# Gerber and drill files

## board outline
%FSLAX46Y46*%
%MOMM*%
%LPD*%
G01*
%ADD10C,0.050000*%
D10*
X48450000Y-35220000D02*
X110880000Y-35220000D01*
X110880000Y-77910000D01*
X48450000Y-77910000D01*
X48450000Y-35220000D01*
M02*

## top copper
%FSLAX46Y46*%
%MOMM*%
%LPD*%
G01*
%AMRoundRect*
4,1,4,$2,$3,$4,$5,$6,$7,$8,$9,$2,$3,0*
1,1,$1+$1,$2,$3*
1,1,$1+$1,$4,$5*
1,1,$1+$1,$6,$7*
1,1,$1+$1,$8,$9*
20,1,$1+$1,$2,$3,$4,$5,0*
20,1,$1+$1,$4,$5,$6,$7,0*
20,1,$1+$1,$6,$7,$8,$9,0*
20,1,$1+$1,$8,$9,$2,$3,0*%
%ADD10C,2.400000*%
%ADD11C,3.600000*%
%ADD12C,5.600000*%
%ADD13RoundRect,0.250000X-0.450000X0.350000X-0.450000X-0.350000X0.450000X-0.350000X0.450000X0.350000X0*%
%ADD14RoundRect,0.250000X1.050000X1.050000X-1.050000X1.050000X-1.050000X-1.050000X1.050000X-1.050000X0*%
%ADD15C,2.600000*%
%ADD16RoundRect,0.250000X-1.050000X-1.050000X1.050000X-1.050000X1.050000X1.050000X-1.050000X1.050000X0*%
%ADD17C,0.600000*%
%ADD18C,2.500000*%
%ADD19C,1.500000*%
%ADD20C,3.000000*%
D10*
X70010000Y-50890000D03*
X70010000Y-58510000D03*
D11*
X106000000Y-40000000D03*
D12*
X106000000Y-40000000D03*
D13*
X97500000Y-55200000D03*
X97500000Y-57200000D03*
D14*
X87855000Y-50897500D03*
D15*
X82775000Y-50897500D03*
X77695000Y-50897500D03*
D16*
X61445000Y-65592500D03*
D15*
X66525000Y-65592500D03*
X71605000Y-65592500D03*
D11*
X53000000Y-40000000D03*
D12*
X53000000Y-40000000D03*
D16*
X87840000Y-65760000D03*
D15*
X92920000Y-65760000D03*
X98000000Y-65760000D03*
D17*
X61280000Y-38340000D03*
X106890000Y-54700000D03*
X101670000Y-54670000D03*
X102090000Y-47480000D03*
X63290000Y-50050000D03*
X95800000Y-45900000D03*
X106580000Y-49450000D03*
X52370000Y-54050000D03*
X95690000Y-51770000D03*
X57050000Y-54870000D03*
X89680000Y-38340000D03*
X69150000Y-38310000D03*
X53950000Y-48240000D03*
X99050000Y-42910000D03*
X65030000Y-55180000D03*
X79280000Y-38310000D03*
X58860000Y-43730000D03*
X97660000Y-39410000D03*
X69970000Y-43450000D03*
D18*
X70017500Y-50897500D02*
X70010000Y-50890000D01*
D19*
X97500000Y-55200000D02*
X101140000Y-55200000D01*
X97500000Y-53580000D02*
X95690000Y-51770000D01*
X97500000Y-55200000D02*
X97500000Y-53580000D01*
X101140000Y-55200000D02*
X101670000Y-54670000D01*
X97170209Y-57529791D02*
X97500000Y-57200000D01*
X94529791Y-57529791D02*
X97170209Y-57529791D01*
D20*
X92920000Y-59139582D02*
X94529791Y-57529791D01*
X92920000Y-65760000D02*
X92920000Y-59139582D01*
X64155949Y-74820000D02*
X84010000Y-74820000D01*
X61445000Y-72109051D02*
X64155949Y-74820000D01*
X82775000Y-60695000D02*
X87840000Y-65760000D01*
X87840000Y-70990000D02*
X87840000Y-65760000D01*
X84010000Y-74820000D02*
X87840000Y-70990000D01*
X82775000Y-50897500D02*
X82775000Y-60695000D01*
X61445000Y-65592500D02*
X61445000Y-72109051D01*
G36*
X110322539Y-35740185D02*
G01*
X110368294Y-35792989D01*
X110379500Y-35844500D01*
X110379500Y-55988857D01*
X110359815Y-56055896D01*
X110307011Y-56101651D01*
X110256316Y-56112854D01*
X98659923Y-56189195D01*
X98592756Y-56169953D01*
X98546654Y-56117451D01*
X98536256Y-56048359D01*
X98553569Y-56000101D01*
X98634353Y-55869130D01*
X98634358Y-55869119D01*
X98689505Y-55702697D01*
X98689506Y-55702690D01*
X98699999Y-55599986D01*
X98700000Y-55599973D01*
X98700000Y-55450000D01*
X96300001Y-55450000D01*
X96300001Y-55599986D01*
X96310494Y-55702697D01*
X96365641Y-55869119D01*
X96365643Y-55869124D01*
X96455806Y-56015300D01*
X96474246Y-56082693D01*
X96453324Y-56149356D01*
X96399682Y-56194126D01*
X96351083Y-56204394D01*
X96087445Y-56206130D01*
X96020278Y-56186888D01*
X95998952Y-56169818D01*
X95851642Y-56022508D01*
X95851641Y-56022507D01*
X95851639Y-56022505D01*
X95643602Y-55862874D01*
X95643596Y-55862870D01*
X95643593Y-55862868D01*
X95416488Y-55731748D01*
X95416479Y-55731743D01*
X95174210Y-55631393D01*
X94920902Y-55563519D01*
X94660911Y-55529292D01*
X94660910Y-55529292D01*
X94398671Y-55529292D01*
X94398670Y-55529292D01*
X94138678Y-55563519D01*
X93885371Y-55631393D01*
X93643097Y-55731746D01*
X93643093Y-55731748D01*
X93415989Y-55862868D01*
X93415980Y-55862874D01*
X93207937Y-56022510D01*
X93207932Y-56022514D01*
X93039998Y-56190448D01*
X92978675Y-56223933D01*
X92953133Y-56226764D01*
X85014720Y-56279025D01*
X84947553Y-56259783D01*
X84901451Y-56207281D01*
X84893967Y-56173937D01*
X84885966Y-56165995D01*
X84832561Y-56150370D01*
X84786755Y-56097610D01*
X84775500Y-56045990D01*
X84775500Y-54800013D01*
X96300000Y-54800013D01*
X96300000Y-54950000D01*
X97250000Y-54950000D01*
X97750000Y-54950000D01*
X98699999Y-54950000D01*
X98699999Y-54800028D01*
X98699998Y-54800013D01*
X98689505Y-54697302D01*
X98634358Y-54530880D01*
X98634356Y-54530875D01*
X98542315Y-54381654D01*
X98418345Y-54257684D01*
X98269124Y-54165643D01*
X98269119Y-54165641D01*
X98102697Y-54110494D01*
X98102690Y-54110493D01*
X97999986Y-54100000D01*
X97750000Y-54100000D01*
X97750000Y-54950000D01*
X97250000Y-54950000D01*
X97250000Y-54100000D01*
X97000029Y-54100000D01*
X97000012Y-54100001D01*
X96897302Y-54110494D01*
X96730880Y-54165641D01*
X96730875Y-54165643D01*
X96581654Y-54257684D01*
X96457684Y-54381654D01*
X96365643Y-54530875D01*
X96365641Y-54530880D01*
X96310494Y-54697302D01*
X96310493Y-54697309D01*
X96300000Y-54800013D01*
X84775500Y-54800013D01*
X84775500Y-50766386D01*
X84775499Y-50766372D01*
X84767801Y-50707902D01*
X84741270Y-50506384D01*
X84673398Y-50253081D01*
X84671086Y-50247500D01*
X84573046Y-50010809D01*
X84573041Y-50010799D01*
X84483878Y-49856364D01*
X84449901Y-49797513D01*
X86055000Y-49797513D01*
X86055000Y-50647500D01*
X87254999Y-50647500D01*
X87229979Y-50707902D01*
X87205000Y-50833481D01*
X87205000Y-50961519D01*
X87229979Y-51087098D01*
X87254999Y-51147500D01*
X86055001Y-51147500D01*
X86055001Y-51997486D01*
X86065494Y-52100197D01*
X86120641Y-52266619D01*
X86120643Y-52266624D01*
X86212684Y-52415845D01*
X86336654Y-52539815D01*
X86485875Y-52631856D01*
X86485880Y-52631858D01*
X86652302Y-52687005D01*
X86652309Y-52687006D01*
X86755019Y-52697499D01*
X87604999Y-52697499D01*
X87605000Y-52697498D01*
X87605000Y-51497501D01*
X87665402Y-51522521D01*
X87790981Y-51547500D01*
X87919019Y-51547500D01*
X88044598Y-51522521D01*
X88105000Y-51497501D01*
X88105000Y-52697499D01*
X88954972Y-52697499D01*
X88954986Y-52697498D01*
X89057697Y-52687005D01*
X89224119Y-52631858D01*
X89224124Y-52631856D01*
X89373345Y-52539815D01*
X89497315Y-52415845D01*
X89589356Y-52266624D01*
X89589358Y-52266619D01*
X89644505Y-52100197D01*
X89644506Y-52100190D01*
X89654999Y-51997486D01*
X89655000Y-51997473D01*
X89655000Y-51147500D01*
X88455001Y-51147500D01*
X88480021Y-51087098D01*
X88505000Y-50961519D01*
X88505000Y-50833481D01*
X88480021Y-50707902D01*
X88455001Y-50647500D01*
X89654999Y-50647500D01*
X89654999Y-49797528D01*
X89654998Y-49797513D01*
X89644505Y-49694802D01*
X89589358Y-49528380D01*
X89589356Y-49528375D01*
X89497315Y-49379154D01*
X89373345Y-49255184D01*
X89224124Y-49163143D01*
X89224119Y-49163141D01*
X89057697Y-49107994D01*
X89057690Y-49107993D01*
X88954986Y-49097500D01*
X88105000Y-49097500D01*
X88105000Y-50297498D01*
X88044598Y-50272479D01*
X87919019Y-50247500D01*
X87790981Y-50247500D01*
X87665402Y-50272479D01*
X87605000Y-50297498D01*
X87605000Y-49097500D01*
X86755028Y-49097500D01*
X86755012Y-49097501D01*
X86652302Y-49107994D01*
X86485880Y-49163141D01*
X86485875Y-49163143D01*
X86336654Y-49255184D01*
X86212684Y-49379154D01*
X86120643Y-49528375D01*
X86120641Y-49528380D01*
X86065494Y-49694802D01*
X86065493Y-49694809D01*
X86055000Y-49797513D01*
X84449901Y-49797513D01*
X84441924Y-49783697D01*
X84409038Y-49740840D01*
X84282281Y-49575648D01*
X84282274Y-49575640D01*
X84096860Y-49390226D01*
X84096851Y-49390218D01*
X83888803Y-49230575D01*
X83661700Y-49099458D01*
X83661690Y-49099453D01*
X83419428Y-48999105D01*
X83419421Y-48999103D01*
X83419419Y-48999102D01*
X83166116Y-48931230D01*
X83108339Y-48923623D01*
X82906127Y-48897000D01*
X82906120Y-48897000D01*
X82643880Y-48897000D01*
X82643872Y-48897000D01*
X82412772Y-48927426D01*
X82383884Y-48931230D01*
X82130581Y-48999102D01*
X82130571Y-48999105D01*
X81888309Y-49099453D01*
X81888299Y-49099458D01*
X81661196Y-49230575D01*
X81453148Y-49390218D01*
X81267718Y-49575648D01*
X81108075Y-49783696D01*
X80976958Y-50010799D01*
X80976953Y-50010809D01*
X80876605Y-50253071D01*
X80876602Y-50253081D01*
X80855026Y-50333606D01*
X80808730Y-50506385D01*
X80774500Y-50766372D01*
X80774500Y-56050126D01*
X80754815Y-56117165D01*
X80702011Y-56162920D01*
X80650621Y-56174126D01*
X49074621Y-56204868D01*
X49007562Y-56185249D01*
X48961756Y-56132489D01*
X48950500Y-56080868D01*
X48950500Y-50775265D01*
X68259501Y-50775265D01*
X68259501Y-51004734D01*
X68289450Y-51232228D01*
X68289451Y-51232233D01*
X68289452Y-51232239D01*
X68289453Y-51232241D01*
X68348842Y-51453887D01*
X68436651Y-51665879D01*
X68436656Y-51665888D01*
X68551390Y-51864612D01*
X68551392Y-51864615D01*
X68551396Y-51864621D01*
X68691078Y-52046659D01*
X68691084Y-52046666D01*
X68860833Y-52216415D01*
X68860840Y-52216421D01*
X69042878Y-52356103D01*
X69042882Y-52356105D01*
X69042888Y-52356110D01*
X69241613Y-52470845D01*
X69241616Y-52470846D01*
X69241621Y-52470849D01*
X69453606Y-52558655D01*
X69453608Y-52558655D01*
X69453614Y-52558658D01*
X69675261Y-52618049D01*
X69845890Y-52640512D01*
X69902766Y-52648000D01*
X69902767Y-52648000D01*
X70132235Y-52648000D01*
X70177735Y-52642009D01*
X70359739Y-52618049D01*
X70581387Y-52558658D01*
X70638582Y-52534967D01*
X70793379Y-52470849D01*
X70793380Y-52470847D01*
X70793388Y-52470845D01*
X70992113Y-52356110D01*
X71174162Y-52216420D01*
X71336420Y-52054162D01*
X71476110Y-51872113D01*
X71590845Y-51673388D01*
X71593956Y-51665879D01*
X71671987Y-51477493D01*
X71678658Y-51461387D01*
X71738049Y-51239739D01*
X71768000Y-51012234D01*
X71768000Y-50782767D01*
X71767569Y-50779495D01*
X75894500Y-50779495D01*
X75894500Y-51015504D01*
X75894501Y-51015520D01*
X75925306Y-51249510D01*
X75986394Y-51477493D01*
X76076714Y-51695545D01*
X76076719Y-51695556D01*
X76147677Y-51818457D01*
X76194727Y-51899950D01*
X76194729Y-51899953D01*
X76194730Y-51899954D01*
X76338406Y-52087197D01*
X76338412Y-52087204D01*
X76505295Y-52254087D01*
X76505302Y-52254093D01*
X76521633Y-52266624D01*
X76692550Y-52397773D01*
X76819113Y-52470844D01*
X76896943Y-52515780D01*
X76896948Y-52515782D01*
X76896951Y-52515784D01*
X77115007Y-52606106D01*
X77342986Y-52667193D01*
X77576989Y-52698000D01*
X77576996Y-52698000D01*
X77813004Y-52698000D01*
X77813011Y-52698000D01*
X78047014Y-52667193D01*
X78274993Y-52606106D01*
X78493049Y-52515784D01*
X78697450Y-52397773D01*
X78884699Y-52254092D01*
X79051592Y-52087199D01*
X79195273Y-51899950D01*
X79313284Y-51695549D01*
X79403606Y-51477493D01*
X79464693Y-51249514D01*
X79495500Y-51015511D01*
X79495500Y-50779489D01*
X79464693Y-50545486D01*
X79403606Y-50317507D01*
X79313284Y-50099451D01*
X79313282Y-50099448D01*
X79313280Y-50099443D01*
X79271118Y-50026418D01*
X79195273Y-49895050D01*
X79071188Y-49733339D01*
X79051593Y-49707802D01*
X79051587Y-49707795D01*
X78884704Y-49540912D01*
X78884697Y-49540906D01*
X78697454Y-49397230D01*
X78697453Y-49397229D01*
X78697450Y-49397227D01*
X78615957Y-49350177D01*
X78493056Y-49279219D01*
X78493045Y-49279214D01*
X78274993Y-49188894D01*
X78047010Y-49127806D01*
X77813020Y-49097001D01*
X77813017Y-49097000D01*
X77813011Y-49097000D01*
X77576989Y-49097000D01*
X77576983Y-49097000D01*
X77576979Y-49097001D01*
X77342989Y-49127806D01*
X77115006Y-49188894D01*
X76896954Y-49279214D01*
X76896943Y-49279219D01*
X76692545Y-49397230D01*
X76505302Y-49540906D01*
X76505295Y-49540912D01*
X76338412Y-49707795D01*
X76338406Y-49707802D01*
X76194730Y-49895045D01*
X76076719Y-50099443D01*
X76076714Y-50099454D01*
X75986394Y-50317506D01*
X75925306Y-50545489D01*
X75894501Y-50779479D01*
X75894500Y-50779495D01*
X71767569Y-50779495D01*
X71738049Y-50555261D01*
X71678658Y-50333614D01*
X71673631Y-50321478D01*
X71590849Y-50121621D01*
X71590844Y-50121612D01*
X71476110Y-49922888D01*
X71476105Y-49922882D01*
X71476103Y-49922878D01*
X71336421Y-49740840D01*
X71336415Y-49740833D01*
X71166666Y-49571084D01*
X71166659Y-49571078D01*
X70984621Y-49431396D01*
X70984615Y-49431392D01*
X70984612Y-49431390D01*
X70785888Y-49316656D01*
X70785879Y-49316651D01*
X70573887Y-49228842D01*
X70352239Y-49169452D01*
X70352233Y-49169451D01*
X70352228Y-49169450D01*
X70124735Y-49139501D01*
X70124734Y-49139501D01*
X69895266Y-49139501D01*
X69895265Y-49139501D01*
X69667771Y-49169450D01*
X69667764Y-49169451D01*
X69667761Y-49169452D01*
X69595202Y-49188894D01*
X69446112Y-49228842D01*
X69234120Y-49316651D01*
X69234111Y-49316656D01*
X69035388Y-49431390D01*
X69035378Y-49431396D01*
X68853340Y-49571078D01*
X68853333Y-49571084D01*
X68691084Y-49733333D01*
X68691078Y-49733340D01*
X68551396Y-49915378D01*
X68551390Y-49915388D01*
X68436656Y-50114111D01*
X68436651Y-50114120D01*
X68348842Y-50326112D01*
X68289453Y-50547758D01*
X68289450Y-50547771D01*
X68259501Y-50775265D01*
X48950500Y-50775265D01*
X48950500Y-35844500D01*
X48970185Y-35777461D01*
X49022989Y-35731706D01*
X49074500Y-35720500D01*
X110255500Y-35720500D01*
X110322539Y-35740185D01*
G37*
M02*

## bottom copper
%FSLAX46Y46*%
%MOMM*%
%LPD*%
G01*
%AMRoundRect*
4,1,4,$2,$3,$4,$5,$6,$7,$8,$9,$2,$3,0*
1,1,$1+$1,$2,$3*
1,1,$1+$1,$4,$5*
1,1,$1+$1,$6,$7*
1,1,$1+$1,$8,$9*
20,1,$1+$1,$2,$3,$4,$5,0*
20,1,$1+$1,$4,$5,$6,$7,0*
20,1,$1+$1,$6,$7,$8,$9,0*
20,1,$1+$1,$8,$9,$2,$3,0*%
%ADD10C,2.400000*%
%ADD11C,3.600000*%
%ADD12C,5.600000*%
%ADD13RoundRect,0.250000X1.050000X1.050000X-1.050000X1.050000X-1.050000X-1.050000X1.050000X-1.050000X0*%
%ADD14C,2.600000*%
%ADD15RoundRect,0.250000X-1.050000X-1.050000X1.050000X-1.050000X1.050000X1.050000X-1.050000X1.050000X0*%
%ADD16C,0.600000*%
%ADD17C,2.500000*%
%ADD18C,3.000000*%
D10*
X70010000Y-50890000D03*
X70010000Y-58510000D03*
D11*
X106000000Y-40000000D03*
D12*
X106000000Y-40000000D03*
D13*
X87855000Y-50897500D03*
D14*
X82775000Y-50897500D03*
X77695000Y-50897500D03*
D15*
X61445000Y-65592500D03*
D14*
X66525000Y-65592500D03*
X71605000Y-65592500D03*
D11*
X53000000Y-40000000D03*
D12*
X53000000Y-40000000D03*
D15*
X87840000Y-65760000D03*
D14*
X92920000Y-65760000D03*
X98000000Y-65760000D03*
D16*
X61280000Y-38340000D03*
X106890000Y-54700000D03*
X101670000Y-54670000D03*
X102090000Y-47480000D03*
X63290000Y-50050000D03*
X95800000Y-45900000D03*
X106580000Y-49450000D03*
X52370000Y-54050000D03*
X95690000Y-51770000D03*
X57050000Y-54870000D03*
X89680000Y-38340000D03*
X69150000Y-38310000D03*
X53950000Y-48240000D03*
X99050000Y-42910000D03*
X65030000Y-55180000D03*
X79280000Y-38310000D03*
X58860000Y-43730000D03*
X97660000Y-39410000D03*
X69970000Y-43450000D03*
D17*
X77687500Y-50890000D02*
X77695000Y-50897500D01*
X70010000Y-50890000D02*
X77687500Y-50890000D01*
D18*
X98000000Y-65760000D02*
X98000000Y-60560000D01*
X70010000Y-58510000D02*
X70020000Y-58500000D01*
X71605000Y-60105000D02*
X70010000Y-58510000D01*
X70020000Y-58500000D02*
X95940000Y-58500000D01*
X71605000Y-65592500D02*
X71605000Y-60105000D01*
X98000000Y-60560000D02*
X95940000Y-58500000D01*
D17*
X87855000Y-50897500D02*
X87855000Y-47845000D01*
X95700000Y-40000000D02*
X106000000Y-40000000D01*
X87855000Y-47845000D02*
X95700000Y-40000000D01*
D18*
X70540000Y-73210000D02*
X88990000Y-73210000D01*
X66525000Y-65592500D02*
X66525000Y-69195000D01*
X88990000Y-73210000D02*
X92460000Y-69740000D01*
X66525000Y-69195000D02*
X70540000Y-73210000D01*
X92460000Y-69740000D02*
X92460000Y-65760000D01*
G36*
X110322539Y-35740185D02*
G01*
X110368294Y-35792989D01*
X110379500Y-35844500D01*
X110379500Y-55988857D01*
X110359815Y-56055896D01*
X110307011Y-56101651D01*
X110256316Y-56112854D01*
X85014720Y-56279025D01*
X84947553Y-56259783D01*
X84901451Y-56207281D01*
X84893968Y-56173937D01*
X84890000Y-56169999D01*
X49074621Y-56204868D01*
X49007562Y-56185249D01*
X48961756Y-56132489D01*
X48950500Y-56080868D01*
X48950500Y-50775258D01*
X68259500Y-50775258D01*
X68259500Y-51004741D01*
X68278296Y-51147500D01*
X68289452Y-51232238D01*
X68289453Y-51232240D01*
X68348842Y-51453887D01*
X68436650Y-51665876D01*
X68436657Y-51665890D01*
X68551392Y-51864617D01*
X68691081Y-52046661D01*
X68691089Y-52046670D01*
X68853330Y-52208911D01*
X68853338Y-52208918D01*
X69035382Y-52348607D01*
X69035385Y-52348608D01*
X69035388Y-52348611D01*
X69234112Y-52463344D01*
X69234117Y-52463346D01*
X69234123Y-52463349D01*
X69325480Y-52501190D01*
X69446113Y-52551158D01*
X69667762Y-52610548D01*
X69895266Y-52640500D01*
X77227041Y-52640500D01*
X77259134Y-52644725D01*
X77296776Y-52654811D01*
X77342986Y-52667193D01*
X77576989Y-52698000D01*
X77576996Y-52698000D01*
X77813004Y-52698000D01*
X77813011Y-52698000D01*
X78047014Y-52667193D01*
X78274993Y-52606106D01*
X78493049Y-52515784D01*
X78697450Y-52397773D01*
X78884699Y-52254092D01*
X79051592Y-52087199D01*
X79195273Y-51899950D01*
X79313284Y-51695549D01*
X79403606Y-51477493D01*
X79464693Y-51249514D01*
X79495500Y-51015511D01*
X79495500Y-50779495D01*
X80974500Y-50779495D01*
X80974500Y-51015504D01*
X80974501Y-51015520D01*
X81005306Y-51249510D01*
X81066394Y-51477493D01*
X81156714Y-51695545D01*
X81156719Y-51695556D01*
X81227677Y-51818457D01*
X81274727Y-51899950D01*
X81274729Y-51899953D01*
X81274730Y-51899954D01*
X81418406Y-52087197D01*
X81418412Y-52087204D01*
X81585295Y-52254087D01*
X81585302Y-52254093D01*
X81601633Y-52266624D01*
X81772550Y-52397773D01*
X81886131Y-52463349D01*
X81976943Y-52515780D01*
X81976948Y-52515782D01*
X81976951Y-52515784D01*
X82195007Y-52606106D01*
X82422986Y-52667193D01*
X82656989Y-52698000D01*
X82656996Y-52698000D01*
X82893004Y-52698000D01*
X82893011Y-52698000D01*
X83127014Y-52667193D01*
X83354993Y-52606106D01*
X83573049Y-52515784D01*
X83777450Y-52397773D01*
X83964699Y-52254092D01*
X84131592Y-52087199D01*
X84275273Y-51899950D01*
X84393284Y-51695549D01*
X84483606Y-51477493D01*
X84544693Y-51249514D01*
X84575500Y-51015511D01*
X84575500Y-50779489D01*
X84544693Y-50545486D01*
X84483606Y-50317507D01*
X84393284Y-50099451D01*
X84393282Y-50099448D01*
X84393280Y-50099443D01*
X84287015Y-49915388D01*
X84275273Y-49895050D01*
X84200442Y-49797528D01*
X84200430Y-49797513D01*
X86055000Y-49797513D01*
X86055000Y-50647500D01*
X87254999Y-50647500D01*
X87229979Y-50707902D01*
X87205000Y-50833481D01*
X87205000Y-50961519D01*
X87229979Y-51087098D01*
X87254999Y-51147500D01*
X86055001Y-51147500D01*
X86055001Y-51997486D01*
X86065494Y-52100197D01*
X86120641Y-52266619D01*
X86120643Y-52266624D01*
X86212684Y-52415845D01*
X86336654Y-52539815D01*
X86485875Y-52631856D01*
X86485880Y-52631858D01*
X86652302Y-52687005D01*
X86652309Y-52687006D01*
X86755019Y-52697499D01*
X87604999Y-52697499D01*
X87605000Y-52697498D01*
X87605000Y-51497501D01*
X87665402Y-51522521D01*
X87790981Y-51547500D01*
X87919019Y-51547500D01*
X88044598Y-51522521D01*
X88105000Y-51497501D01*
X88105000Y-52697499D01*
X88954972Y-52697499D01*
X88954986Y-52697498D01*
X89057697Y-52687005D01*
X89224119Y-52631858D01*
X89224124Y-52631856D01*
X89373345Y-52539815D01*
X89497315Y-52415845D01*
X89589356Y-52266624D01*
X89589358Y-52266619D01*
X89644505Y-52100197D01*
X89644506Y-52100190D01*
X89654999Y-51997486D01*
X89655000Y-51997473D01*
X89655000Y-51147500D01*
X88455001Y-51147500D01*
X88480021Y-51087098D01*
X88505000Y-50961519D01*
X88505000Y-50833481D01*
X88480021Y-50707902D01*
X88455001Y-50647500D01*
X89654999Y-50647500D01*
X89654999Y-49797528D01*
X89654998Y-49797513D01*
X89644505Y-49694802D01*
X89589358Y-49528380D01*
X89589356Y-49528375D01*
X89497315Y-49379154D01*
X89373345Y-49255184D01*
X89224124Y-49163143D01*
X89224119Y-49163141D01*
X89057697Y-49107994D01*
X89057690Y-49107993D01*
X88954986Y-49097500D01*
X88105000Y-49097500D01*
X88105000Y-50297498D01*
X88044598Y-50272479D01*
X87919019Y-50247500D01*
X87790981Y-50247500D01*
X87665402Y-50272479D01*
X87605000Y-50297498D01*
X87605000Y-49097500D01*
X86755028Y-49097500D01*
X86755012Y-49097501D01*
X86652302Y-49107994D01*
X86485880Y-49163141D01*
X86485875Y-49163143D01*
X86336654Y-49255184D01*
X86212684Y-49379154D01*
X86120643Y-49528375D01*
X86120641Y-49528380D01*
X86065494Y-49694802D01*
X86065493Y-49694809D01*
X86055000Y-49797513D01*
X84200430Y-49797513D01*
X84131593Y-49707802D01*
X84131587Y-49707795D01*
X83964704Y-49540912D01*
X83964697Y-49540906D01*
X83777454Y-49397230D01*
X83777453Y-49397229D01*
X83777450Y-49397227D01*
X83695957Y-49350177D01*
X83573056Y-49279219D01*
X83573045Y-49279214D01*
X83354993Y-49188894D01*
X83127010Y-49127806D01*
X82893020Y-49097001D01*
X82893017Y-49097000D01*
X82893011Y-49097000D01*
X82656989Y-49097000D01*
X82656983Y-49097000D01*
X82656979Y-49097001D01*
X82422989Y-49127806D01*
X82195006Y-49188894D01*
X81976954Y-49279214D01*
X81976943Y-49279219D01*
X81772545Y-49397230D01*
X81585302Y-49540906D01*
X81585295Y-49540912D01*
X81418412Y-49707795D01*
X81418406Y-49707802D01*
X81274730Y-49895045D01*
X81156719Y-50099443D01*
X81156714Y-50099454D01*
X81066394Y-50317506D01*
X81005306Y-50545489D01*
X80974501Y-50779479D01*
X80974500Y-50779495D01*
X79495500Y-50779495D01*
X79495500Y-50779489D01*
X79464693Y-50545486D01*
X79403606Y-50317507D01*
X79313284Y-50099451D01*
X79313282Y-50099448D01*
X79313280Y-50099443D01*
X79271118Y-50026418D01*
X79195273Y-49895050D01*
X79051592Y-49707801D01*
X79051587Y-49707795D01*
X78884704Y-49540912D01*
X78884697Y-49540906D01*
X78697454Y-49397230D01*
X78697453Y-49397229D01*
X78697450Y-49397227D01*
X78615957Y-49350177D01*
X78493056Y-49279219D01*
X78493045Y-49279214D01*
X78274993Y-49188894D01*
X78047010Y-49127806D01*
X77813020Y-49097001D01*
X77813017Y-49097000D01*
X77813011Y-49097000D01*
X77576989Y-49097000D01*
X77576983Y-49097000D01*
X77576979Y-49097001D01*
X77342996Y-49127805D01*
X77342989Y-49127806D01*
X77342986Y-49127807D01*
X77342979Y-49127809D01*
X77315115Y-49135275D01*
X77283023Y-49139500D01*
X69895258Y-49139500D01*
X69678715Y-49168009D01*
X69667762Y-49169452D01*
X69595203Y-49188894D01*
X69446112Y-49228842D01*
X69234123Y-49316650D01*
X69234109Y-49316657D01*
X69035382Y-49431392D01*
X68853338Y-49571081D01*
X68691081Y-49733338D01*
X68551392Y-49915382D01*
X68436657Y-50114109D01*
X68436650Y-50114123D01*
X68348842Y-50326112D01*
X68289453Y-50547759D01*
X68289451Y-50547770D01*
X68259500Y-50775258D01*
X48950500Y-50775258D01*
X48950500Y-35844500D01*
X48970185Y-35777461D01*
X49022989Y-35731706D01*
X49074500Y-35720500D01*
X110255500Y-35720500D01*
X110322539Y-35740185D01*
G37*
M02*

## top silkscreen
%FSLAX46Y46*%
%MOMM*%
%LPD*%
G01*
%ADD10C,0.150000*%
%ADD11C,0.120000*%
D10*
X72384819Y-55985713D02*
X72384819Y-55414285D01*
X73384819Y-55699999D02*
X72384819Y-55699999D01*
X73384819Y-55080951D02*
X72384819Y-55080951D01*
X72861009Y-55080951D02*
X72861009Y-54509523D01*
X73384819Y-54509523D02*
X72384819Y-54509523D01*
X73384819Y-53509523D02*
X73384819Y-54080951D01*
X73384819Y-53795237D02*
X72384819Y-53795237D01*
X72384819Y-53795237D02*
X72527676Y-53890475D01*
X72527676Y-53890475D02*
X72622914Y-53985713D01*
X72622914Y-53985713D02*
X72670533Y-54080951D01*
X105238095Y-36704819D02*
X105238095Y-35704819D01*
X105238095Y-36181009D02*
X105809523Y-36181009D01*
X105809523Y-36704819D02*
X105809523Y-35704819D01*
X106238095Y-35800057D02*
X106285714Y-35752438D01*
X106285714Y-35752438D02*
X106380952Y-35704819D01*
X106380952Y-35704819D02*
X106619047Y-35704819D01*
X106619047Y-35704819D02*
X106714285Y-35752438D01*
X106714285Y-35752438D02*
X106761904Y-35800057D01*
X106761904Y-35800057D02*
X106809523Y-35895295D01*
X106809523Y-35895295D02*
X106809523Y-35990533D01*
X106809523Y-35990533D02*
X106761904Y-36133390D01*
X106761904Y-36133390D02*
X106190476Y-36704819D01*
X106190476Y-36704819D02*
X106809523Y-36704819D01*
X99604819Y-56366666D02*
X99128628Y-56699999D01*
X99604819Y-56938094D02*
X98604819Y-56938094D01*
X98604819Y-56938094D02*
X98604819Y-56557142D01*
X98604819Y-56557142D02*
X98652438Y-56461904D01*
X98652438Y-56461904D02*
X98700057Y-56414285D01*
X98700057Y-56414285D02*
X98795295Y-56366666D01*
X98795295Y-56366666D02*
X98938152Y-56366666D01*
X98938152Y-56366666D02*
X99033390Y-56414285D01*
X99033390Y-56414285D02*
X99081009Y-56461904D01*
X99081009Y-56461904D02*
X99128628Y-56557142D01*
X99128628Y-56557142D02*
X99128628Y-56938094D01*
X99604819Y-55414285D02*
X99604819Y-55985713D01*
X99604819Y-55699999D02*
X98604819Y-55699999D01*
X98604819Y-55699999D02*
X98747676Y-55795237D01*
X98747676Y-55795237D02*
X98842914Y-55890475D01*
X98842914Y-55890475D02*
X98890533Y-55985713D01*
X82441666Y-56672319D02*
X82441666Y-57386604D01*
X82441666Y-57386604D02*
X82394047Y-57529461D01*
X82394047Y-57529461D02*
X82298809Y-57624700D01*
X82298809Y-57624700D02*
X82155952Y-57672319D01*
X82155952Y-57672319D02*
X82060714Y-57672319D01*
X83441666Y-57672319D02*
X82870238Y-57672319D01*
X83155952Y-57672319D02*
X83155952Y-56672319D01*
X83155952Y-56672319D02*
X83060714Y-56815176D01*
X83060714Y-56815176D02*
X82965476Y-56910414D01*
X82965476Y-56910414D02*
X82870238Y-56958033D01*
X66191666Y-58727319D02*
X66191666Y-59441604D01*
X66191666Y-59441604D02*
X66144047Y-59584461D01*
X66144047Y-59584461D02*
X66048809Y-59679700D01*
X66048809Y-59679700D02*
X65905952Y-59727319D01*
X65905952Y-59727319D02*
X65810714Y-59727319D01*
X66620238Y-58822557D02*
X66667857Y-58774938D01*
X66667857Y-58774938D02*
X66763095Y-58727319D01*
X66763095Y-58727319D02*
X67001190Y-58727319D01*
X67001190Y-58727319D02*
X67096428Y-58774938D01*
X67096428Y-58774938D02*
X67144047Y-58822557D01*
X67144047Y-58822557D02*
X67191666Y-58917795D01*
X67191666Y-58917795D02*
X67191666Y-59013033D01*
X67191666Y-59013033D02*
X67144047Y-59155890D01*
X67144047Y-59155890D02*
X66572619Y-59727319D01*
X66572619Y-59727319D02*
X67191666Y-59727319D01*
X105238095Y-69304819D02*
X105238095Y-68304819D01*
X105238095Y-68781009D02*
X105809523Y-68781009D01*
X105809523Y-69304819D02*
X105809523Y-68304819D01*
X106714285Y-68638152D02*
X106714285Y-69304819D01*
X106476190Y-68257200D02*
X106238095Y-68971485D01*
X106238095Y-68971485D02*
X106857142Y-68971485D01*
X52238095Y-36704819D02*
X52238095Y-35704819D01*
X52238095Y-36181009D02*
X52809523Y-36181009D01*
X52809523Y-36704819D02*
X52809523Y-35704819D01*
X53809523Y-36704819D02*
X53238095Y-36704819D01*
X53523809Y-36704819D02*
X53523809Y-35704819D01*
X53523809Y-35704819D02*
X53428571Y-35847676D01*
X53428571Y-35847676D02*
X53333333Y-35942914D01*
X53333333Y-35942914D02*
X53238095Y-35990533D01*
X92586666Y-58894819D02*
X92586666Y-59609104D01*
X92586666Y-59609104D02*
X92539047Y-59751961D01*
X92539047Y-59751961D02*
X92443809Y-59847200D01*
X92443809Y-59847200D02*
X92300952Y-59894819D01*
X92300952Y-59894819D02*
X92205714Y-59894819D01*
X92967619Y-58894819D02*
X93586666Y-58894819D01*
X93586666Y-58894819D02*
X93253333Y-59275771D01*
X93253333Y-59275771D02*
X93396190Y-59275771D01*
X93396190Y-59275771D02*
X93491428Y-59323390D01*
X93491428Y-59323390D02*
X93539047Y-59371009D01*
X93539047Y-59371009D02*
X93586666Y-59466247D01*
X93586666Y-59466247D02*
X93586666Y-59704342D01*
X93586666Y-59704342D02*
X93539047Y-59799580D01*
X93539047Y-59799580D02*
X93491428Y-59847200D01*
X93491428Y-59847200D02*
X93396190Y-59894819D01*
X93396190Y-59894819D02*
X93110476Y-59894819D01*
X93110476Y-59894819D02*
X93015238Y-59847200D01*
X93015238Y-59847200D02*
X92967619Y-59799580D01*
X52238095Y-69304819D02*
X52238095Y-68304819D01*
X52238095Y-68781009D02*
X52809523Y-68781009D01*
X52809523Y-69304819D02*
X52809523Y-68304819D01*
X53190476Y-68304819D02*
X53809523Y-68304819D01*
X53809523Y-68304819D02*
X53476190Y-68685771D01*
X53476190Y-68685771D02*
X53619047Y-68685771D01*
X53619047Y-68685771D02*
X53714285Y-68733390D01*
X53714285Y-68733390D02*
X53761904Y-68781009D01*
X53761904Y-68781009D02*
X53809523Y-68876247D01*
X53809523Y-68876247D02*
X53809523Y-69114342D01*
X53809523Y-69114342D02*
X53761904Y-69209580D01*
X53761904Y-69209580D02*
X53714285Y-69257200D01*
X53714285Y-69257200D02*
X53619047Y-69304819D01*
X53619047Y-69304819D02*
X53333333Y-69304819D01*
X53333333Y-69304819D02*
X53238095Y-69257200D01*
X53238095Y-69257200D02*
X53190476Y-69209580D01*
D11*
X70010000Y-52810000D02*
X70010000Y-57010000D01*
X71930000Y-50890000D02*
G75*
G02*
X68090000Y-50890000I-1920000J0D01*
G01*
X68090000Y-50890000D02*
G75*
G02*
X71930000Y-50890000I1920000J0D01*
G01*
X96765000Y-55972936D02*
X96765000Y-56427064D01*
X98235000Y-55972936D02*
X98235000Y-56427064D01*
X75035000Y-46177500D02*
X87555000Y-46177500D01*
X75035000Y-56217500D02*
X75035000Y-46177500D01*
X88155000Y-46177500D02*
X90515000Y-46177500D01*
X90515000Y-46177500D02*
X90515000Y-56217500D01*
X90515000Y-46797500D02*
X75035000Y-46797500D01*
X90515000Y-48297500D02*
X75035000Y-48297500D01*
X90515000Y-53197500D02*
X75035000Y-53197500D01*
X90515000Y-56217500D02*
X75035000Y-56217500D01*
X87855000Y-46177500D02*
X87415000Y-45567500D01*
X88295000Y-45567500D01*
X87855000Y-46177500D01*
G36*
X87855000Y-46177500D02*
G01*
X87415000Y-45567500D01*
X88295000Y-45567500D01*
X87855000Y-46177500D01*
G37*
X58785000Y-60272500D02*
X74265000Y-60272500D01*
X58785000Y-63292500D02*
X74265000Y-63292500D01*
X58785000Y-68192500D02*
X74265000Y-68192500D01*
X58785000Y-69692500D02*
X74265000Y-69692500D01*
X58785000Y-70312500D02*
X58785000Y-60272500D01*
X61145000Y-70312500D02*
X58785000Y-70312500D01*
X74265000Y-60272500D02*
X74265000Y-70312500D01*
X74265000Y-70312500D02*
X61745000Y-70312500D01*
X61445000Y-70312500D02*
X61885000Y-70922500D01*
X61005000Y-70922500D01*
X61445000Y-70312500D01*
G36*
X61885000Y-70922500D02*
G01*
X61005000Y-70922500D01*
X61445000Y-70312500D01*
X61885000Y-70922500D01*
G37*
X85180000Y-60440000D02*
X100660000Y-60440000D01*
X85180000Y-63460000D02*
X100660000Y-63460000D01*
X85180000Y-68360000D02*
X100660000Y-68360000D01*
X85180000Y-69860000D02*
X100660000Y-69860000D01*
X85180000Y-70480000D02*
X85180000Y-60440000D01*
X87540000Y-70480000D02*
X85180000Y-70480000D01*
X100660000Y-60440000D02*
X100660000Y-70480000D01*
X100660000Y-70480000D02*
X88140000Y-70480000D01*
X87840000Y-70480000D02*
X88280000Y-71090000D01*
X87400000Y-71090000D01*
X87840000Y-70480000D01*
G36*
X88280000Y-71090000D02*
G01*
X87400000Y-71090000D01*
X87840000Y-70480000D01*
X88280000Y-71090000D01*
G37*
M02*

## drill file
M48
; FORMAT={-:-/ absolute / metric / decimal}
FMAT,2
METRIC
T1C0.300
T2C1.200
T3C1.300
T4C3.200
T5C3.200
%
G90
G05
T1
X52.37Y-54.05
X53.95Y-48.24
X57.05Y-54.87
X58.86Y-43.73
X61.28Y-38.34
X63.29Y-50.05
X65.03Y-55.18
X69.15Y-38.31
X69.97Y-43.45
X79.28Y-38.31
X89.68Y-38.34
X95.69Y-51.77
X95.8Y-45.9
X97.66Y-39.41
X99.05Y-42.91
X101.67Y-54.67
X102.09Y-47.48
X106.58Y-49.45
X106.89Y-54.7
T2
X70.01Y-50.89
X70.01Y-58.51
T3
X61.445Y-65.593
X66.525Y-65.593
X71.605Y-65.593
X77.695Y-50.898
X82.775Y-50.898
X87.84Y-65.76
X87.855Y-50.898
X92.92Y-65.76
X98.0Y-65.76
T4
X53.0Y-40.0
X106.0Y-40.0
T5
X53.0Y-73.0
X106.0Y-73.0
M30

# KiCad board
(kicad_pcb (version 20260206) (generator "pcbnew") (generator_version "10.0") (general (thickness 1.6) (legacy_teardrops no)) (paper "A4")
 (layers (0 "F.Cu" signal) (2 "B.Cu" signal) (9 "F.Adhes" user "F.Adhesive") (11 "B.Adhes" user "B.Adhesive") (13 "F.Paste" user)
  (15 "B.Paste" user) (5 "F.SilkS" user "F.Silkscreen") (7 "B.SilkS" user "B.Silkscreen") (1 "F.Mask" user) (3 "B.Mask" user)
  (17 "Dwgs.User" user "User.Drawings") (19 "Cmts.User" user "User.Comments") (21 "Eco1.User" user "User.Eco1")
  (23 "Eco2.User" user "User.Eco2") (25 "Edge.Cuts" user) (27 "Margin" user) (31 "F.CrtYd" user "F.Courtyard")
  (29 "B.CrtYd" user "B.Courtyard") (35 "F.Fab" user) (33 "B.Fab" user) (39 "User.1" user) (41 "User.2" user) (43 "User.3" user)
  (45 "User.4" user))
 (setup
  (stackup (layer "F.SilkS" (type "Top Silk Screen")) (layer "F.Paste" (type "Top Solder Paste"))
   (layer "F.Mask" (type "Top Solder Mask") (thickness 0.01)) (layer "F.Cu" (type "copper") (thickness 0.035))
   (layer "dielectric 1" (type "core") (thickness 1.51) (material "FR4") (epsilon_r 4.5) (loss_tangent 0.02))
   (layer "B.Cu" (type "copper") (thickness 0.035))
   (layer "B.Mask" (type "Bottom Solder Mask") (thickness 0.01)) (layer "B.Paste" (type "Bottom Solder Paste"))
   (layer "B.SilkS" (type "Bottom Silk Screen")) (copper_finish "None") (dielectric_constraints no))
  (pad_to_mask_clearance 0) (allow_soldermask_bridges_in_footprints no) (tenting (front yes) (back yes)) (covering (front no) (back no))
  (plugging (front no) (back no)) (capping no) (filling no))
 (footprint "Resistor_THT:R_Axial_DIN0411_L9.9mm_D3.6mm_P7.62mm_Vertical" (layer "F.Cu") (at 70.01 50.89 -90)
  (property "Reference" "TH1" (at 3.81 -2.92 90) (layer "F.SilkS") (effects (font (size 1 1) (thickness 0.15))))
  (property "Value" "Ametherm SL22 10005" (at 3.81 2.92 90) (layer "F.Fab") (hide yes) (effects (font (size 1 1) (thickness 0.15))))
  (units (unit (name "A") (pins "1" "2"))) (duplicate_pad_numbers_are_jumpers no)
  (fp_line (start 1.92 0) (end 6.12 0) (stroke (width 0.12) (type solid)) (layer "F.SilkS"))
  (fp_circle (center 0 0) (end 1.92 0) (stroke (width 0.12) (type solid)) (fill no) (layer "F.SilkS"))
  (pad "1" thru_hole circle (at 0 0 270) (size 2.4 2.4) (drill 1.2) (layers "*.Cu" "*.Mask") (remove_unused_layers no) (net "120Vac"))
  (pad "2" thru_hole circle (at 7.62 0 270) (size 2.4 2.4) (drill 1.2) (layers "*.Cu" "*.Mask") (remove_unused_layers no) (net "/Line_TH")))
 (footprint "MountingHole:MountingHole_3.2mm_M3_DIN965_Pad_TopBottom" (layer "F.Cu") (at 106 40)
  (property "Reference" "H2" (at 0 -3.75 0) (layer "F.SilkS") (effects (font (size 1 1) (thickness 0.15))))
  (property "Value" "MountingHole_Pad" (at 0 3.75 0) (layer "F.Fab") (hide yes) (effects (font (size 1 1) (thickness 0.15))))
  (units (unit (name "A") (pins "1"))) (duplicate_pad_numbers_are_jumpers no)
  (pad "1" thru_hole circle (at 0 0) (size 3.6 3.6) (drill 3.2) (layers "*.Cu" "*.Mask") (remove_unused_layers no) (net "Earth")
   (zone_connect 2))
  (pad "1" connect circle (at 0 0) (size 5.6 5.6) (layers "F.Cu" "F.Mask") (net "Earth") (zone_connect 2))
  (pad "1" connect circle (at 0 0) (size 5.6 5.6) (layers "B.Cu" "B.Mask") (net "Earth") (zone_connect 2)))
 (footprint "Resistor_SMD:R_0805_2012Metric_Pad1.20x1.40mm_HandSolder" (layer "F.Cu") (at 97.5 56.2 -90)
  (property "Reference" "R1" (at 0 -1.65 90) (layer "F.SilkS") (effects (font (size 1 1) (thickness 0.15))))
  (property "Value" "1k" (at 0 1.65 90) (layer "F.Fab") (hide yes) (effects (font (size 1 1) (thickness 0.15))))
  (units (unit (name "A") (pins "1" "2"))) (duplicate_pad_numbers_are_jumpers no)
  (fp_line (start -0.227064 0.735) (end 0.227064 0.735) (stroke (width 0.12) (type solid)) (layer "F.SilkS"))
  (fp_line (start -0.227064 -0.735) (end 0.227064 -0.735) (stroke (width 0.12) (type solid)) (layer "F.SilkS"))
  (pad "1" smd roundrect (at -1 0 270) (size 1.2 1.4) (layers "F.Cu" "F.Mask" "F.Paste") (roundrect_rratio 0.208333) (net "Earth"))
  (pad "2" smd roundrect (at 1 0 270) (size 1.2 1.4) (layers "F.Cu" "F.Mask" "F.Paste") (roundrect_rratio 0.208333) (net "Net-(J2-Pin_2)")))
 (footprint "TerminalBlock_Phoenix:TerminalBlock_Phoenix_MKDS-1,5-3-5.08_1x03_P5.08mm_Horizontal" (layer "F.Cu") (at 87.855 50.8975 180)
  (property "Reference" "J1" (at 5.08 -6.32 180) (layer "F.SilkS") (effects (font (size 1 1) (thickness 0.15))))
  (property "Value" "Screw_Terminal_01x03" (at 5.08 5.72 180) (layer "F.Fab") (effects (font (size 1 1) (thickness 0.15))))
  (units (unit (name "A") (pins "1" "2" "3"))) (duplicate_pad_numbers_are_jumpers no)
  (fp_line (start 12.82 4.72) (end 0.3 4.72) (stroke (width 0.12) (type solid)) (layer "F.SilkS"))
  (fp_line (start 12.82 -5.32) (end 12.82 4.72) (stroke (width 0.12) (type solid)) (layer "F.SilkS"))
  (fp_line (start -0.3 4.72) (end -2.66 4.72) (stroke (width 0.12) (type solid)) (layer "F.SilkS"))
  (fp_line (start -2.66 4.72) (end -2.66 -5.32) (stroke (width 0.12) (type solid)) (layer "F.SilkS"))
  (fp_line (start -2.66 4.1) (end 12.82 4.1) (stroke (width 0.12) (type solid)) (layer "F.SilkS"))
  (fp_line (start -2.66 2.6) (end 12.82 2.6) (stroke (width 0.12) (type solid)) (layer "F.SilkS"))
  (fp_line (start -2.66 -2.3) (end 12.82 -2.3) (stroke (width 0.12) (type solid)) (layer "F.SilkS"))
  (fp_line (start -2.66 -5.32) (end 12.82 -5.32) (stroke (width 0.12) (type solid)) (layer "F.SilkS"))
  (fp_poly (pts (xy 0 4.72) (xy 0.44 5.33) (xy -0.44 5.33)) (stroke (width 0.12) (type solid)) (fill yes) (layer "F.SilkS"))
  (pad "1" thru_hole roundrect (at 0 0 180) (size 2.6 2.6) (drill 1.3) (layers "*.Cu" "*.Mask") (remove_unused_layers no)
   (roundrect_rratio 0.096154) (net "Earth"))
  (pad "2" thru_hole circle (at 5.08 0 180) (size 2.6 2.6) (drill 1.3) (layers "*.Cu" "*.Mask") (remove_unused_layers no) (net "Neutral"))
  (pad "3" thru_hole circle (at 10.16 0 180) (size 2.6 2.6) (drill 1.3) (layers "*.Cu" "*.Mask") (remove_unused_layers no) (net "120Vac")))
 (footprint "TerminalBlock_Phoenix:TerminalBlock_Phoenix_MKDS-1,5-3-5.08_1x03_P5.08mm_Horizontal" (layer "F.Cu") (at 61.445 65.5925)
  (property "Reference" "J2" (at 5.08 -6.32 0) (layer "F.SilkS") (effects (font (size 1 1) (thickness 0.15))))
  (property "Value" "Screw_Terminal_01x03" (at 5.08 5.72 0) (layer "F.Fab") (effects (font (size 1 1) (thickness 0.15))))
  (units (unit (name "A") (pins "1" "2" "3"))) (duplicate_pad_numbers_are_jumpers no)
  (fp_line (start -2.66 -5.32) (end 12.82 -5.32) (stroke (width 0.12) (type solid)) (layer "F.SilkS"))
  (fp_line (start -2.66 -2.3) (end 12.82 -2.3) (stroke (width 0.12) (type solid)) (layer "F.SilkS"))
  (fp_line (start -2.66 2.6) (end 12.82 2.6) (stroke (width 0.12) (type solid)) (layer "F.SilkS"))
  (fp_line (start -2.66 4.1) (end 12.82 4.1) (stroke (width 0.12) (type solid)) (layer "F.SilkS"))
  (fp_line (start -2.66 4.72) (end -2.66 -5.32) (stroke (width 0.12) (type solid)) (layer "F.SilkS"))
  (fp_line (start -0.3 4.72) (end -2.66 4.72) (stroke (width 0.12) (type solid)) (layer "F.SilkS"))
  (fp_line (start 12.82 -5.32) (end 12.82 4.72) (stroke (width 0.12) (type solid)) (layer "F.SilkS"))
  (fp_line (start 12.82 4.72) (end 0.3 4.72) (stroke (width 0.12) (type solid)) (layer "F.SilkS"))
  (fp_poly (pts (xy 0 4.72) (xy 0.44 5.33) (xy -0.44 5.33)) (stroke (width 0.12) (type solid)) (fill yes) (layer "F.SilkS"))
  (pad "1" thru_hole roundrect (at 0 0) (size 2.6 2.6) (drill 1.3) (layers "*.Cu" "*.Mask") (remove_unused_layers no)
   (roundrect_rratio 0.096154) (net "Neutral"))
  (pad "2" thru_hole circle (at 5.08 0) (size 2.6 2.6) (drill 1.3) (layers "*.Cu" "*.Mask") (remove_unused_layers no) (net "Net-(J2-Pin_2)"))
  (pad "3" thru_hole circle (at 10.16 0) (size 2.6 2.6) (drill 1.3) (layers "*.Cu" "*.Mask") (remove_unused_layers no) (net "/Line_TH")))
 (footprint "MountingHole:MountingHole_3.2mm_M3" (layer "F.Cu") (at 106 73)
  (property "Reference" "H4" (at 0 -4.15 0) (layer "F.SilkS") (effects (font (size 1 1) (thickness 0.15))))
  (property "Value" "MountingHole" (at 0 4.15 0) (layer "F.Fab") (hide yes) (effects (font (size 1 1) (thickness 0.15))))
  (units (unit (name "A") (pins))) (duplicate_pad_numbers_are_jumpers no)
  (pad "" np_thru_hole circle (at 0 0) (size 3.2 3.2) (drill 3.2) (layers "*.Cu" "*.Mask")))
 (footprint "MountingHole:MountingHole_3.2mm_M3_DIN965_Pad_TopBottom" (layer "F.Cu") (at 53 40)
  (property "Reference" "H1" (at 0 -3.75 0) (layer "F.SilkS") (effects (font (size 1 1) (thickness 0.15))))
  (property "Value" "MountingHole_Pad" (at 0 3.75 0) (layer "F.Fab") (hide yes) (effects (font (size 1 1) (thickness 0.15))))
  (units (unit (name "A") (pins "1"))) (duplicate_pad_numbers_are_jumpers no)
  (pad "1" thru_hole circle (at 0 0) (size 3.6 3.6) (drill 3.2) (layers "*.Cu" "*.Mask") (remove_unused_layers no) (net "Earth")
   (zone_connect 2))
  (pad "1" connect circle (at 0 0) (size 5.6 5.6) (layers "F.Cu" "F.Mask") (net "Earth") (zone_connect 2))
  (pad "1" connect circle (at 0 0) (size 5.6 5.6) (layers "B.Cu" "B.Mask") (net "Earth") (zone_connect 2)))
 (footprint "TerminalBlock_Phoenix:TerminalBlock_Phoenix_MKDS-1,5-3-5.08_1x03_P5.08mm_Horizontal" (layer "F.Cu") (at 87.84 65.76)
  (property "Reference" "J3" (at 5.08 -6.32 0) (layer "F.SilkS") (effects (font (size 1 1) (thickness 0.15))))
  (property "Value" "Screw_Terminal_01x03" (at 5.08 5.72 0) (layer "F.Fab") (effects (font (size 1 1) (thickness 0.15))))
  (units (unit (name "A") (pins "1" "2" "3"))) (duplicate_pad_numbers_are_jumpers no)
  (fp_line (start -2.66 -5.32) (end 12.82 -5.32) (stroke (width 0.12) (type solid)) (layer "F.SilkS"))
  (fp_line (start -2.66 -2.3) (end 12.82 -2.3) (stroke (width 0.12) (type solid)) (layer "F.SilkS"))
  (fp_line (start -2.66 2.6) (end 12.82 2.6) (stroke (width 0.12) (type solid)) (layer "F.SilkS"))
  (fp_line (start -2.66 4.1) (end 12.82 4.1) (stroke (width 0.12) (type solid)) (layer "F.SilkS"))
  (fp_line (start -2.66 4.72) (end -2.66 -5.32) (stroke (width 0.12) (type solid)) (layer "F.SilkS"))
  (fp_line (start -0.3 4.72) (end -2.66 4.72) (stroke (width 0.12) (type solid)) (layer "F.SilkS"))
  (fp_line (start 12.82 -5.32) (end 12.82 4.72) (stroke (width 0.12) (type solid)) (layer "F.SilkS"))
  (fp_line (start 12.82 4.72) (end 0.3 4.72) (stroke (width 0.12) (type solid)) (layer "F.SilkS"))
  (fp_poly (pts (xy 0 4.72) (xy 0.44 5.33) (xy -0.44 5.33)) (stroke (width 0.12) (type solid)) (fill yes) (layer "F.SilkS"))
  (pad "1" thru_hole roundrect (at 0 0) (size 2.6 2.6) (drill 1.3) (layers "*.Cu" "*.Mask") (remove_unused_layers no)
   (roundrect_rratio 0.096154) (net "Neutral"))
  (pad "2" thru_hole circle (at 5.08 0) (size 2.6 2.6) (drill 1.3) (layers "*.Cu" "*.Mask") (remove_unused_layers no) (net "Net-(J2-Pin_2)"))
  (pad "3" thru_hole circle (at 10.16 0) (size 2.6 2.6) (drill 1.3) (layers "*.Cu" "*.Mask") (remove_unused_layers no) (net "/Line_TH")))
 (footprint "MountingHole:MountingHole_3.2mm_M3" (layer "F.Cu") (at 53 73)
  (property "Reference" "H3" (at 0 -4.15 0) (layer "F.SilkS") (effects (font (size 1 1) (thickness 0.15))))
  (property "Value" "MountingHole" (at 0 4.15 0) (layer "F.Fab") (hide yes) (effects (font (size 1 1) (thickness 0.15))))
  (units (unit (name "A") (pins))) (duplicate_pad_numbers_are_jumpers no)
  (pad "" np_thru_hole circle (at 0 0) (size 3.2 3.2) (drill 3.2) (layers "*.Cu" "*.Mask")))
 (gr_rect (start 48.45 35.22) (end 110.88 77.91) (stroke (width 0.05) (type default)) (fill no) (layer "Edge.Cuts"))
 (segment (start 70.0175 50.8975) (end 70.01 50.89) (width 2.5) (layer "F.Cu") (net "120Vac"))
 (segment (start 77.6875 50.89) (end 77.695 50.8975) (width 2.5) (layer "B.Cu") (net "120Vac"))
 (segment (start 70.01 50.89) (end 77.6875 50.89) (width 2.5) (layer "B.Cu") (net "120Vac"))
 (segment (start 98 65.76) (end 98 60.56) (width 3) (layer "B.Cu") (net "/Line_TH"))
 (segment (start 70.01 58.51) (end 70.02 58.5) (width 3) (layer "B.Cu") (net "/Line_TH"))
 (segment (start 71.605 60.105) (end 70.01 58.51) (width 3) (layer "B.Cu") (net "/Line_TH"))
 (segment (start 70.02 58.5) (end 95.94 58.5) (width 3) (layer "B.Cu") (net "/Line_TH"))
 (segment (start 71.605 65.5925) (end 71.605 60.105) (width 3) (layer "B.Cu") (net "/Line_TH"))
 (segment (start 98 60.56) (end 95.94 58.5) (width 3) (layer "B.Cu") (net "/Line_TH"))
 (segment (start 97.5 55.2) (end 101.14 55.2) (width 1.5) (layer "F.Cu") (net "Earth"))
 (segment (start 97.5 53.58) (end 95.69 51.77) (width 1.5) (layer "F.Cu") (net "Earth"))
 (segment (start 97.5 55.2) (end 97.5 53.58) (width 1.5) (layer "F.Cu") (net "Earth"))
 (segment (start 101.14 55.2) (end 101.67 54.67) (width 1.5) (layer "F.Cu") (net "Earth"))
 (via (at 61.28 38.34) (size 0.6) (drill 0.3) (layers "F.Cu" "B.Cu") (free yes) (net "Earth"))
 (via (at 106.89 54.7) (size 0.6) (drill 0.3) (layers "F.Cu" "B.Cu") (free yes) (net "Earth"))
 (via (at 101.67 54.67) (size 0.6) (drill 0.3) (layers "F.Cu" "B.Cu") (free yes) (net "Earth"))
 (via (at 102.09 47.48) (size 0.6) (drill 0.3) (layers "F.Cu" "B.Cu") (free yes) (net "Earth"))
 (via (at 63.29 50.05) (size 0.6) (drill 0.3) (layers "F.Cu" "B.Cu") (free yes) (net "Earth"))
 (via (at 95.8 45.9) (size 0.6) (drill 0.3) (layers "F.Cu" "B.Cu") (free yes) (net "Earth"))
 (via (at 106.58 49.45) (size 0.6) (drill 0.3) (layers "F.Cu" "B.Cu") (free yes) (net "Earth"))
 (via (at 52.37 54.05) (size 0.6) (drill 0.3) (layers "F.Cu" "B.Cu") (free yes) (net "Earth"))
 (via (at 95.69 51.77) (size 0.6) (drill 0.3) (layers "F.Cu" "B.Cu") (free yes) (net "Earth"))
 (via (at 57.05 54.87) (size 0.6) (drill 0.3) (layers "F.Cu" "B.Cu") (free yes) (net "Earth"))
 (via (at 89.68 38.34) (size 0.6) (drill 0.3) (layers "F.Cu" "B.Cu") (free yes) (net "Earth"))
 (via (at 69.15 38.31) (size 0.6) (drill 0.3) (layers "F.Cu" "B.Cu") (free yes) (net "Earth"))
 (via (at 53.95 48.24) (size 0.6) (drill 0.3) (layers "F.Cu" "B.Cu") (free yes) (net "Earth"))
 (via (at 99.05 42.91) (size 0.6) (drill 0.3) (layers "F.Cu" "B.Cu") (free yes) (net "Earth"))
 (via (at 65.03 55.18) (size 0.6) (drill 0.3) (layers "F.Cu" "B.Cu") (free yes) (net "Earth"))
 (via (at 79.28 38.31) (size 0.6) (drill 0.3) (layers "F.Cu" "B.Cu") (free yes) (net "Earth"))
 (via (at 58.86 43.73) (size 0.6) (drill 0.3) (layers "F.Cu" "B.Cu") (free yes) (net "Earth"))
 (via (at 97.66 39.41) (size 0.6) (drill 0.3) (layers "F.Cu" "B.Cu") (free yes) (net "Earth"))
 (via (at 69.97 43.45) (size 0.6) (drill 0.3) (layers "F.Cu" "B.Cu") (free yes) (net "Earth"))
 (segment (start 87.855 50.8975) (end 87.855 47.845) (width 2.5) (layer "B.Cu") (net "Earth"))
 (segment (start 95.7 40) (end 106 40) (width 2.5) (layer "B.Cu") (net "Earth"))
 (segment (start 87.855 47.845) (end 95.7 40) (width 2.5) (layer "B.Cu") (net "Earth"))
 (segment (start 97.170209 57.529791) (end 97.5 57.2) (width 1.5) (layer "F.Cu") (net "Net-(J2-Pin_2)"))
 (segment (start 94.529791 57.529791) (end 97.170209 57.529791) (width 1.5) (layer "F.Cu") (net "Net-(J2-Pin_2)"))
 (segment (start 92.92 59.139582) (end 94.529791 57.529791) (width 3) (layer "F.Cu") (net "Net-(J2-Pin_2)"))
 (segment (start 92.92 65.76) (end 92.92 59.139582) (width 3) (layer "F.Cu") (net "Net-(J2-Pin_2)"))
 (segment (start 70.54 73.21) (end 88.99 73.21) (width 3) (layer "B.Cu") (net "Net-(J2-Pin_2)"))
 (segment (start 66.525 65.5925) (end 66.525 69.195) (width 3) (layer "B.Cu") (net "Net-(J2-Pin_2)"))
 (segment (start 88.99 73.21) (end 92.46 69.74) (width 3) (layer "B.Cu") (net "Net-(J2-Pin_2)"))
 (segment (start 66.525 69.195) (end 70.54 73.21) (width 3) (layer "B.Cu") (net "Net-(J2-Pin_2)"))
 (segment (start 92.46 69.74) (end 92.46 65.76) (width 3) (layer "B.Cu") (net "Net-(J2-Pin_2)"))
 (segment (start 64.155949 74.82) (end 84.01 74.82) (width 3) (layer "F.Cu") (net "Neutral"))
 (segment (start 61.445 72.109051) (end 64.155949 74.82) (width 3) (layer "F.Cu") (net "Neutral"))
 (segment (start 82.775 60.695) (end 87.84 65.76) (width 3) (layer "F.Cu") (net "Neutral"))
 (segment (start 87.84 70.99) (end 87.84 65.76) (width 3) (layer "F.Cu") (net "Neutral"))
 (segment (start 84.01 74.82) (end 87.84 70.99) (width 3) (layer "F.Cu") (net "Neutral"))
 (segment (start 82.775 50.8975) (end 82.775 60.695) (width 3) (layer "F.Cu") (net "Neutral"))
 (segment (start 61.445 65.5925) (end 61.445 72.109051) (width 3) (layer "F.Cu") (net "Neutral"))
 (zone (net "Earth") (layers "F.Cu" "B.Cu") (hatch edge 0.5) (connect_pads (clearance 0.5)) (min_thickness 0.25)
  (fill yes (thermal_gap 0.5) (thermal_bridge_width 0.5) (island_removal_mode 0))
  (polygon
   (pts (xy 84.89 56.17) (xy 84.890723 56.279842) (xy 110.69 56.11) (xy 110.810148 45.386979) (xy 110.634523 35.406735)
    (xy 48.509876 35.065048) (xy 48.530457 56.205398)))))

